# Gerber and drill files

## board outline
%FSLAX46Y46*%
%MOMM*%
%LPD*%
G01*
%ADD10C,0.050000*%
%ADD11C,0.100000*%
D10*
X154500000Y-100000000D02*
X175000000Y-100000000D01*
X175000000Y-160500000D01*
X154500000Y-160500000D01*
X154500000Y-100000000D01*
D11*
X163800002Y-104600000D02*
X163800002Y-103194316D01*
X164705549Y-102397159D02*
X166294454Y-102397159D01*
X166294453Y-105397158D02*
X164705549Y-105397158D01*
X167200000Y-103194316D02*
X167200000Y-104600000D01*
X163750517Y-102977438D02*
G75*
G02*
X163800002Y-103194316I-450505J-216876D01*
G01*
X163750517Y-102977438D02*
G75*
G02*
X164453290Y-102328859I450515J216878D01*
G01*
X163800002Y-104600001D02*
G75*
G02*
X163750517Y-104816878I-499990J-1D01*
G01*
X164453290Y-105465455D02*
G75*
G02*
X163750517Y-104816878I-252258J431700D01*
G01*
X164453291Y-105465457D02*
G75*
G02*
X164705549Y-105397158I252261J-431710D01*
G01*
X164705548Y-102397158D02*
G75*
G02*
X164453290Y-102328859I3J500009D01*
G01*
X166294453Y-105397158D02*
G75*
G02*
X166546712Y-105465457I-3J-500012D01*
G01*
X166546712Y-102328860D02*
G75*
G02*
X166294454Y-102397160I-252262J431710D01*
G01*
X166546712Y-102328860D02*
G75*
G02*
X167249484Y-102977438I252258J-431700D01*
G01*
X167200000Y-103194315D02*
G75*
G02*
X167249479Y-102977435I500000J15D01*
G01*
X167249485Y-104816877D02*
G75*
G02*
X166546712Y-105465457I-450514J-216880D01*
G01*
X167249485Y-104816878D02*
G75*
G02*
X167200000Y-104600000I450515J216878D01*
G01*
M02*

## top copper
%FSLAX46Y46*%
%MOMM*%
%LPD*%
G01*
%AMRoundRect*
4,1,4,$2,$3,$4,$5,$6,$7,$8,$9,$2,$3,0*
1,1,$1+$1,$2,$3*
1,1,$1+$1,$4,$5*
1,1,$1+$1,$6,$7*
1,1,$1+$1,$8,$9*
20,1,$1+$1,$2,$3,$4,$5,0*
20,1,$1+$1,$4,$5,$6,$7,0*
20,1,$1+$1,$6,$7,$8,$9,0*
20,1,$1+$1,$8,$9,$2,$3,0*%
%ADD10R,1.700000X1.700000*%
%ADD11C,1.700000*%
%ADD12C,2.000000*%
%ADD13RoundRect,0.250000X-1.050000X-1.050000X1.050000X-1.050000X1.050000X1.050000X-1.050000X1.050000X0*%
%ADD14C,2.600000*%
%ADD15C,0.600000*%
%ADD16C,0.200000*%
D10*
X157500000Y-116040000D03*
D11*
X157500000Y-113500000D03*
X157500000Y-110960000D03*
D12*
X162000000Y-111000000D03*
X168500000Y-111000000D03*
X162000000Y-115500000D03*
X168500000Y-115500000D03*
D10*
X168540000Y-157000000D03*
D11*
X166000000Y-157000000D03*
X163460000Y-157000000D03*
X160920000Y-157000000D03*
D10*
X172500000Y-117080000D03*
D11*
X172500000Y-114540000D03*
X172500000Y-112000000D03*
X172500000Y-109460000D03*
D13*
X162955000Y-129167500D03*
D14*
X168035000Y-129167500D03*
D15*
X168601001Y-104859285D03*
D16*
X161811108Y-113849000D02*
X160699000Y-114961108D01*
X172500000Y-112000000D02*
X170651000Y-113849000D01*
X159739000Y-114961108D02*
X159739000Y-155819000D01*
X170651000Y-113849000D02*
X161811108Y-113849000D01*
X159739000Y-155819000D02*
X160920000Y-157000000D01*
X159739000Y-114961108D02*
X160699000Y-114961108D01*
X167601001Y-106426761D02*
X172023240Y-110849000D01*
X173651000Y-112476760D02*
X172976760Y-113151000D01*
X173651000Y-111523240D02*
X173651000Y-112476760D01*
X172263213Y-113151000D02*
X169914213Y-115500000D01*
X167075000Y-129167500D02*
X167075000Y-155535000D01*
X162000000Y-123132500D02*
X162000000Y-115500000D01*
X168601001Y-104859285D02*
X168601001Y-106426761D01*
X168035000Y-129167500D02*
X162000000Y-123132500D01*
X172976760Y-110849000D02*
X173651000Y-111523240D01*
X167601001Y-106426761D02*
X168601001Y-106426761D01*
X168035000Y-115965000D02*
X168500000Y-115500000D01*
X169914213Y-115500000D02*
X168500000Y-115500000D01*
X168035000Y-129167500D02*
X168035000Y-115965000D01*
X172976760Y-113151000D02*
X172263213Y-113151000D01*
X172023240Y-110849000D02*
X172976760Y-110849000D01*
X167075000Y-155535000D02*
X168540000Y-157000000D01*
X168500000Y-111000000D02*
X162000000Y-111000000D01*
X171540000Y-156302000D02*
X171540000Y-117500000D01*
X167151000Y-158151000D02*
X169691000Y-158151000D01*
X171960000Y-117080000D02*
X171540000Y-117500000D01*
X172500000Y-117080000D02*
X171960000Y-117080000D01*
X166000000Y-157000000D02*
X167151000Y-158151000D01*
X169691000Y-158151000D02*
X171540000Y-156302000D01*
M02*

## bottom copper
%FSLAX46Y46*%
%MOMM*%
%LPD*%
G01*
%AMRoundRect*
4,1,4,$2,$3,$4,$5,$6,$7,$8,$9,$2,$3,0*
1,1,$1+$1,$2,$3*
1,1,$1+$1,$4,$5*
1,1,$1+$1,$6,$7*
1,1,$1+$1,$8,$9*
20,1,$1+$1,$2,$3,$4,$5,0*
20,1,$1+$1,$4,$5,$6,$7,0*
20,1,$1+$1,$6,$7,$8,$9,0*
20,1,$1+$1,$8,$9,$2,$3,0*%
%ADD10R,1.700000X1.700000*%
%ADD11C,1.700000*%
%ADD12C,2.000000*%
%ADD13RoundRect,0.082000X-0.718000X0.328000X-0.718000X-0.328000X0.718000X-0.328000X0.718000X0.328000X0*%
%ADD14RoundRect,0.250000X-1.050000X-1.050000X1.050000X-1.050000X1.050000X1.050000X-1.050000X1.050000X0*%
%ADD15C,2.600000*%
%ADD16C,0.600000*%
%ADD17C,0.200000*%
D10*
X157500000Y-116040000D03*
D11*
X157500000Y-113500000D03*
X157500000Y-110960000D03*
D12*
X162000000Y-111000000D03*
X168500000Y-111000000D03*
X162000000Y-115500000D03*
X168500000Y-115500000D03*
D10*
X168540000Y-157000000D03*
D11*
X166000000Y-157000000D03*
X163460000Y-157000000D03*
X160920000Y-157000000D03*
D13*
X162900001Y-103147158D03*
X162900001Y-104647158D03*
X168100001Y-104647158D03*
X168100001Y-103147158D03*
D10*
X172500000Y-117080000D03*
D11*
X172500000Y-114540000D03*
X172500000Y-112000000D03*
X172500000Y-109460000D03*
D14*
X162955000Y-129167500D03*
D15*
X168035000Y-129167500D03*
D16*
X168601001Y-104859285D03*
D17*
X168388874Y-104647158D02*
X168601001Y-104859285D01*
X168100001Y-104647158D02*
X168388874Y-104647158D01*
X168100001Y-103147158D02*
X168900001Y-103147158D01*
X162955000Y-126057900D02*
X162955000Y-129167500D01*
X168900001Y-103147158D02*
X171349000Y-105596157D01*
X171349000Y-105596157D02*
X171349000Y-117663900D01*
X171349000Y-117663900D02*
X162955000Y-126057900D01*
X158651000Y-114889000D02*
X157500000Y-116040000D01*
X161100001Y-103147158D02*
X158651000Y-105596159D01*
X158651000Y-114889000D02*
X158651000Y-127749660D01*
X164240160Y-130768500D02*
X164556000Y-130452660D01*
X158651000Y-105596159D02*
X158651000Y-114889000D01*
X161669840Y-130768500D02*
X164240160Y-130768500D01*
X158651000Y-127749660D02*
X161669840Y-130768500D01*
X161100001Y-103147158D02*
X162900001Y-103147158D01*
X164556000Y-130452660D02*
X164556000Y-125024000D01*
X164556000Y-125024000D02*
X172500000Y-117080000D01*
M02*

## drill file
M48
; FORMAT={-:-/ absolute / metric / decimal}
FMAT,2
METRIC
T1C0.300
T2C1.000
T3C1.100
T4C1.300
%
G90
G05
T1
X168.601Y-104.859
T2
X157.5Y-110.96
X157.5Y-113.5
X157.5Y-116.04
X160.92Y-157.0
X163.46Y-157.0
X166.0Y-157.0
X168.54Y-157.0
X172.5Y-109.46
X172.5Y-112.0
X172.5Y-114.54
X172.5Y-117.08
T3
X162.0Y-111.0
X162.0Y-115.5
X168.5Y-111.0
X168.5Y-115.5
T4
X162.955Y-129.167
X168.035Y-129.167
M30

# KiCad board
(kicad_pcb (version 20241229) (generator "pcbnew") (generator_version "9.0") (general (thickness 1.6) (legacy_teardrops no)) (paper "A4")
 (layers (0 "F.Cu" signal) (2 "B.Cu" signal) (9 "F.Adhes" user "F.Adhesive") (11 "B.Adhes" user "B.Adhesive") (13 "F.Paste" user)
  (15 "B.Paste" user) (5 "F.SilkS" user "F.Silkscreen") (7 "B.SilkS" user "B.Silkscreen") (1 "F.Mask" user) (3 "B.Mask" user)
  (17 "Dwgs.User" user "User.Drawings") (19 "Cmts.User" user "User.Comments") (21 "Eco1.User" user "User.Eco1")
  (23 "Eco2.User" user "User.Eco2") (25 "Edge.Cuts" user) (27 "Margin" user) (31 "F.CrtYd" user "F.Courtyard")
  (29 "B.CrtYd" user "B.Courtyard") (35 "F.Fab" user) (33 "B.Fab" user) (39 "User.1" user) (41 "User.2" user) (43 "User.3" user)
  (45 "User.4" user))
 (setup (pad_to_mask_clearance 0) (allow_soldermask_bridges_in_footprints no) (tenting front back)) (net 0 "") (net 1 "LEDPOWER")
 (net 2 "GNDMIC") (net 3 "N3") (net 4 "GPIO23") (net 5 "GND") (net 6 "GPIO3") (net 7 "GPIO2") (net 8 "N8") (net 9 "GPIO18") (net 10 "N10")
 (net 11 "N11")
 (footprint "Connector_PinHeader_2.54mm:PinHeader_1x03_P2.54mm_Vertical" (layer "F.Cu") (at 157.5 116.04 180)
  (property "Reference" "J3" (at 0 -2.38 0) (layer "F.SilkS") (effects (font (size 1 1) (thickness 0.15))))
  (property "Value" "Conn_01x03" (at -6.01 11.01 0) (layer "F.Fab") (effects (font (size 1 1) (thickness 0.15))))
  (pad "1" thru_hole rect (at 0 0 180) (size 1.7 1.7) (drill 1) (layers "*.Cu" "*.Mask") (remove_unused_layers no) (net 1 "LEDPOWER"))
  (pad "2" thru_hole circle (at 0 2.54 180) (size 1.7 1.7) (drill 1) (layers "*.Cu" "*.Mask") (remove_unused_layers no) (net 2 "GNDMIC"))
  (pad "3" thru_hole circle (at 0 5.08 180) (size 1.7 1.7) (drill 1) (layers "*.Cu" "*.Mask") (remove_unused_layers no) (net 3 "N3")))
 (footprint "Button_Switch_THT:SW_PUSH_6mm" (layer "F.Cu") (at 162 111)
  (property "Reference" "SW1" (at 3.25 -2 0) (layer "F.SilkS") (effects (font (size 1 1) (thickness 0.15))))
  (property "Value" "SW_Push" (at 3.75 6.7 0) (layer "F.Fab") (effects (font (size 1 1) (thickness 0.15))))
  (pad "1" thru_hole circle (at 0 0 90) (size 2 2) (drill 1.1) (layers "*.Cu" "*.Mask") (remove_unused_layers no) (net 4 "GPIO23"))
  (pad "1" thru_hole circle (at 6.5 0 90) (size 2 2) (drill 1.1) (layers "*.Cu" "*.Mask") (remove_unused_layers no) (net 4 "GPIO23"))
  (pad "2" thru_hole circle (at 0 4.5 90) (size 2 2) (drill 1.1) (layers "*.Cu" "*.Mask") (remove_unused_layers no) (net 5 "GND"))
  (pad "2" thru_hole circle (at 6.5 4.5 90) (size 2 2) (drill 1.1) (layers "*.Cu" "*.Mask") (remove_unused_layers no) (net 5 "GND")))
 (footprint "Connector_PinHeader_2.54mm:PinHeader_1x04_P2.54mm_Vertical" (layer "F.Cu") (at 168.54 157 -90)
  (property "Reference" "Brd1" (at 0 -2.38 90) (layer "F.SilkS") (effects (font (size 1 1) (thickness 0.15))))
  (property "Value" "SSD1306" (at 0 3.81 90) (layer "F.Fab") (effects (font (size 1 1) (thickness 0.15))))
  (pad "1" thru_hole rect (at 0 0 270) (size 1.7 1.7) (drill 1) (layers "*.Cu" "*.Mask") (remove_unused_layers no) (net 5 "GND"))
  (pad "2" thru_hole circle (at 0 2.54 270) (size 1.7 1.7) (drill 1) (layers "*.Cu" "*.Mask") (remove_unused_layers no) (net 1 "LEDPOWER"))
  (pad "3" thru_hole circle (at 0 5.08 270) (size 1.7 1.7) (drill 1) (layers "*.Cu" "*.Mask") (remove_unused_layers no) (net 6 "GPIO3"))
  (pad "4" thru_hole circle (at 0 7.62 270) (size 1.7 1.7) (drill 1) (layers "*.Cu" "*.Mask") (remove_unused_layers no) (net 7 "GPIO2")))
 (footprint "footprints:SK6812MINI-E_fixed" (layer "F.Cu") (at 165.5 104)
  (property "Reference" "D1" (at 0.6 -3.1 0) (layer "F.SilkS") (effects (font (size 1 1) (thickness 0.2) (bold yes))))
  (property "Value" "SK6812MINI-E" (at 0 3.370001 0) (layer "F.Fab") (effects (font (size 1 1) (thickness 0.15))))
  (fp_line (start -1.699998 0.6) (end -1.699998 -0.805684) (stroke (width 0.1) (type solid)) (layer "Edge.Cuts"))
  (fp_line (start -0.794451 -1.602841) (end 0.794454 -1.602841) (stroke (width 0.1) (type solid)) (layer "Edge.Cuts"))
  (fp_line (start 0.794453 1.397158) (end -0.794451 1.397158) (stroke (width 0.1) (type solid)) (layer "Edge.Cuts"))
  (fp_line (start 1.7 -0.805684) (end 1.7 0.6) (stroke (width 0.1) (type solid)) (layer "Edge.Cuts"))
  (fp_arc (start -1.749483 -1.022562) (mid -1.712526 -0.91691) (end -1.699998 -0.805684) (stroke (width 0.1) (type solid))
   (layer "Edge.Cuts"))
  (fp_arc (start -1.749483 -1.022562) (mid -1.63807 -1.606877) (end -1.04671 -1.671141) (stroke (width 0.1) (type solid))
   (layer "Edge.Cuts"))
  (fp_arc (start -1.699998 0.600001) (mid -1.712526 0.711226) (end -1.749483 0.816878) (stroke (width 0.1) (type solid)) (layer "Edge.Cuts"))
  (fp_arc (start -1.04671 1.465455) (mid -1.638069 1.401192) (end -1.749483 0.816878) (stroke (width 0.1) (type solid)) (layer "Edge.Cuts"))
  (fp_arc (start -1.046709 1.465457) (mid -0.925121 1.414535) (end -0.794451 1.397158) (stroke (width 0.1) (type solid)) (layer "Edge.Cuts"))
  (fp_arc (start -0.794452 -1.602842) (mid -0.925122 -1.620219) (end -1.04671 -1.671141) (stroke (width 0.1) (type solid))
   (layer "Edge.Cuts"))
  (fp_arc (start 0.794453 1.397158) (mid 0.925124 1.414535) (end 1.046712 1.465457) (stroke (width 0.1) (type solid)) (layer "Edge.Cuts"))
  (fp_arc (start 1.046712 -1.67114) (mid 0.925124 -1.620218) (end 0.794454 -1.602841) (stroke (width 0.1) (type solid)) (layer "Edge.Cuts"))
  (fp_arc (start 1.046712 -1.67114) (mid 1.638072 -1.606876) (end 1.749485 -1.022562) (stroke (width 0.1) (type solid)) (layer "Edge.Cuts"))
  (fp_arc (start 1.7 -0.805685) (mid 1.712528 -0.91691) (end 1.749485 -1.022562) (stroke (width 0.1) (type solid)) (layer "Edge.Cuts"))
  (fp_arc (start 1.749485 0.816877) (mid 1.638073 1.401193) (end 1.046712 1.465457) (stroke (width 0.1) (type solid)) (layer "Edge.Cuts"))
  (fp_arc (start 1.749485 0.816878) (mid 1.712528 0.711226) (end 1.7 0.6) (stroke (width 0.1) (type solid)) (layer "Edge.Cuts"))
  (pad "1" smd roundrect (at -2.599999 -0.852842 270) (size 0.82 1.6) (layers "B.Cu" "B.Mask" "B.Paste") (roundrect_rratio 0.1)
   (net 1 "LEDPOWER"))
  (pad "2" smd roundrect (at -2.599999 0.647158 270) (size 0.82 1.6) (layers "B.Cu" "B.Mask" "B.Paste") (roundrect_rratio 0.1) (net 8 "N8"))
  (pad "3" smd roundrect (at 2.600001 0.647158 270) (size 0.82 1.6) (layers "B.Cu" "B.Mask" "B.Paste") (roundrect_rratio 0.1) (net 5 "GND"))
  (pad "4" smd roundrect (at 2.600001 -0.852842 270) (size 0.82 1.6) (layers "B.Cu" "B.Mask" "B.Paste") (roundrect_rratio 0.1)
   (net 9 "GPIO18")))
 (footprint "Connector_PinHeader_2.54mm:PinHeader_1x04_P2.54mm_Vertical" (layer "F.Cu") (at 172.5 117.08 180)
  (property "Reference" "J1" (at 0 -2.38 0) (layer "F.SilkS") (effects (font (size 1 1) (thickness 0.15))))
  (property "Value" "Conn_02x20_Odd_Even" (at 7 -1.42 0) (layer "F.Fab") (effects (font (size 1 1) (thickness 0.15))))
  (pad "1" thru_hole rect (at 0 0 180) (size 1.7 1.7) (drill 1) (layers "*.Cu" "*.Mask") (remove_unused_layers no) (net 1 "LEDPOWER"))
  (pad "2" thru_hole circle (at 0 2.54 180) (size 1.7 1.7) (drill 1) (layers "*.Cu" "*.Mask") (remove_unused_layers no) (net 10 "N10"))
  (pad "3" thru_hole circle (at 0 5.08 180) (size 1.7 1.7) (drill 1) (layers "*.Cu" "*.Mask") (remove_unused_layers no) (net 7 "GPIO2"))
  (pad "4" thru_hole circle (at 0 7.62 180) (size 1.7 1.7) (drill 1) (layers "*.Cu" "*.Mask") (remove_unused_layers no) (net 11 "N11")))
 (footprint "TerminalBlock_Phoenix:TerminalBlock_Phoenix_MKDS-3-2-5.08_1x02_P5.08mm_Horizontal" (layer "F.Cu") (at 162.955 129.1675)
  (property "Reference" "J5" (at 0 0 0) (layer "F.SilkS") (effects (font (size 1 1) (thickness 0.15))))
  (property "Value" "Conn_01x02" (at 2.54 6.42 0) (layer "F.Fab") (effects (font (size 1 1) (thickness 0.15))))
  (pad "1" thru_hole roundrect (at 0 0) (size 2.6 2.6) (drill 1.3) (layers "*.Cu" "*.Mask") (remove_unused_layers no)
   (roundrect_rratio 0.096154) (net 9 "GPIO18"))
  (pad "2" thru_hole circle (at 5.08 0) (size 2.6 2.6) (drill 1.3) (layers "*.Cu" "*.Mask") (remove_unused_layers no) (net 5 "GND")))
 (gr_rect (start 154.5 100) (end 175 160.5) (stroke (width 0.05) (type default)) (fill no) (layer "Edge.Cuts"))
 (segment (start 161.811108 113.849) (end 160.699 114.961108) (width 0.2) (layer "F.Cu") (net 7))
 (segment (start 172.5 112) (end 170.651 113.849) (width 0.2) (layer "F.Cu") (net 7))
 (segment (start 159.739 114.961108) (end 159.739 155.819) (width 0.2) (layer "F.Cu") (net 7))
 (segment (start 170.651 113.849) (end 161.811108 113.849) (width 0.2) (layer "F.Cu") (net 7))
 (segment (start 159.739 155.819) (end 160.92 157) (width 0.2) (layer "F.Cu") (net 7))
 (segment (start 159.739 114.961108) (end 160.699 114.961108) (width 0.2) (layer "F.Cu") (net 7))
 (segment (start 167.601001 106.426761) (end 172.02324 110.849) (width 0.2) (layer "F.Cu") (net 5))
 (segment (start 173.651 112.47676) (end 172.97676 113.151) (width 0.2) (layer "F.Cu") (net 5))
 (segment (start 173.651 111.52324) (end 173.651 112.47676) (width 0.2) (layer "F.Cu") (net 5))
 (segment (start 172.263213 113.151) (end 169.914213 115.5) (width 0.2) (layer "F.Cu") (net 5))
 (segment (start 167.075 129.1675) (end 167.075 155.535) (width 0.2) (layer "F.Cu") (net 5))
 (segment (start 162 123.1325) (end 162 115.5) (width 0.2) (layer "F.Cu") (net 5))
 (segment (start 168.601001 104.859285) (end 168.601001 106.426761) (width 0.2) (layer "F.Cu") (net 5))
 (segment (start 168.035 129.1675) (end 162 123.1325) (width 0.2) (layer "F.Cu") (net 5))
 (segment (start 172.97676 110.849) (end 173.651 111.52324) (width 0.2) (layer "F.Cu") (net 5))
 (segment (start 167.601001 106.426761) (end 168.601001 106.426761) (width 0.2) (layer "F.Cu") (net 5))
 (segment (start 168.035 115.965) (end 168.5 115.5) (width 0.2) (layer "F.Cu") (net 5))
 (segment (start 169.914213 115.5) (end 168.5 115.5) (width 0.2) (layer "F.Cu") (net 5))
 (segment (start 168.035 129.1675) (end 168.035 115.965) (width 0.2) (layer "F.Cu") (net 5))
 (segment (start 172.97676 113.151) (end 172.263213 113.151) (width 0.2) (layer "F.Cu") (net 5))
 (segment (start 172.02324 110.849) (end 172.97676 110.849) (width 0.2) (layer "F.Cu") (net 5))
 (segment (start 167.075 155.535) (end 168.54 157) (width 0.2) (layer "F.Cu") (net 5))
 (via (at 168.601001 104.859285) (size 0.6) (drill 0.3) (layers "F.Cu" "B.Cu") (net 5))
 (segment (start 168.388874 104.647158) (end 168.601001 104.859285) (width 0.2) (layer "B.Cu") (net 5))
 (segment (start 168.100001 104.647158) (end 168.388874 104.647158) (width 0.2) (layer "B.Cu") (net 5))
 (segment (start 168.100001 103.147158) (end 168.900001 103.147158) (width 0.2) (layer "B.Cu") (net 9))
 (segment (start 162.955 126.0579) (end 162.955 129.1675) (width 0.2) (layer "B.Cu") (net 9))
 (segment (start 168.900001 103.147158) (end 171.349 105.596157) (width 0.2) (layer "B.Cu") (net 9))
 (segment (start 171.349 105.596157) (end 171.349 117.6639) (width 0.2) (layer "B.Cu") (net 9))
 (segment (start 171.349 117.6639) (end 162.955 126.0579) (width 0.2) (layer "B.Cu") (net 9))
 (segment (start 168.5 111) (end 162 111) (width 0.2) (layer "F.Cu") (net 4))
 (segment (start 171.54 156.302) (end 171.54 117.5) (width 0.2) (layer "F.Cu") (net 1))
 (segment (start 167.151 158.151) (end 169.691 158.151) (width 0.2) (layer "F.Cu") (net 1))
 (segment (start 171.96 117.08) (end 171.54 117.5) (width 0.2) (layer "F.Cu") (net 1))
 (segment (start 172.5 117.08) (end 171.96 117.08) (width 0.2) (layer "F.Cu") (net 1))
 (segment (start 166 157) (end 167.151 158.151) (width 0.2) (layer "F.Cu") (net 1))
 (segment (start 169.691 158.151) (end 171.54 156.302) (width 0.2) (layer "F.Cu") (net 1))
 (segment (start 158.651 114.889) (end 157.5 116.04) (width 0.2) (layer "B.Cu") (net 1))
 (segment (start 161.100001 103.147158) (end 158.651 105.596159) (width 0.2) (layer "B.Cu") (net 1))
 (segment (start 158.651 114.889) (end 158.651 127.74966) (width 0.2) (layer "B.Cu") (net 1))
 (segment (start 164.24016 130.7685) (end 164.556 130.45266) (width 0.2) (layer "B.Cu") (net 1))
 (segment (start 158.651 105.596159) (end 158.651 114.889) (width 0.2) (layer "B.Cu") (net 1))
 (segment (start 161.66984 130.7685) (end 164.24016 130.7685) (width 0.2) (layer "B.Cu") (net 1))
 (segment (start 158.651 127.74966) (end 161.66984 130.7685) (width 0.2) (layer "B.Cu") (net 1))
 (segment (start 161.100001 103.147158) (end 162.900001 103.147158) (width 0.2) (layer "B.Cu") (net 1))
 (segment (start 164.556 130.45266) (end 164.556 125.024) (width 0.2) (layer "B.Cu") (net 1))
 (segment (start 164.556 125.024) (end 172.5 117.08) (width 0.2) (layer "B.Cu") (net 1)))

